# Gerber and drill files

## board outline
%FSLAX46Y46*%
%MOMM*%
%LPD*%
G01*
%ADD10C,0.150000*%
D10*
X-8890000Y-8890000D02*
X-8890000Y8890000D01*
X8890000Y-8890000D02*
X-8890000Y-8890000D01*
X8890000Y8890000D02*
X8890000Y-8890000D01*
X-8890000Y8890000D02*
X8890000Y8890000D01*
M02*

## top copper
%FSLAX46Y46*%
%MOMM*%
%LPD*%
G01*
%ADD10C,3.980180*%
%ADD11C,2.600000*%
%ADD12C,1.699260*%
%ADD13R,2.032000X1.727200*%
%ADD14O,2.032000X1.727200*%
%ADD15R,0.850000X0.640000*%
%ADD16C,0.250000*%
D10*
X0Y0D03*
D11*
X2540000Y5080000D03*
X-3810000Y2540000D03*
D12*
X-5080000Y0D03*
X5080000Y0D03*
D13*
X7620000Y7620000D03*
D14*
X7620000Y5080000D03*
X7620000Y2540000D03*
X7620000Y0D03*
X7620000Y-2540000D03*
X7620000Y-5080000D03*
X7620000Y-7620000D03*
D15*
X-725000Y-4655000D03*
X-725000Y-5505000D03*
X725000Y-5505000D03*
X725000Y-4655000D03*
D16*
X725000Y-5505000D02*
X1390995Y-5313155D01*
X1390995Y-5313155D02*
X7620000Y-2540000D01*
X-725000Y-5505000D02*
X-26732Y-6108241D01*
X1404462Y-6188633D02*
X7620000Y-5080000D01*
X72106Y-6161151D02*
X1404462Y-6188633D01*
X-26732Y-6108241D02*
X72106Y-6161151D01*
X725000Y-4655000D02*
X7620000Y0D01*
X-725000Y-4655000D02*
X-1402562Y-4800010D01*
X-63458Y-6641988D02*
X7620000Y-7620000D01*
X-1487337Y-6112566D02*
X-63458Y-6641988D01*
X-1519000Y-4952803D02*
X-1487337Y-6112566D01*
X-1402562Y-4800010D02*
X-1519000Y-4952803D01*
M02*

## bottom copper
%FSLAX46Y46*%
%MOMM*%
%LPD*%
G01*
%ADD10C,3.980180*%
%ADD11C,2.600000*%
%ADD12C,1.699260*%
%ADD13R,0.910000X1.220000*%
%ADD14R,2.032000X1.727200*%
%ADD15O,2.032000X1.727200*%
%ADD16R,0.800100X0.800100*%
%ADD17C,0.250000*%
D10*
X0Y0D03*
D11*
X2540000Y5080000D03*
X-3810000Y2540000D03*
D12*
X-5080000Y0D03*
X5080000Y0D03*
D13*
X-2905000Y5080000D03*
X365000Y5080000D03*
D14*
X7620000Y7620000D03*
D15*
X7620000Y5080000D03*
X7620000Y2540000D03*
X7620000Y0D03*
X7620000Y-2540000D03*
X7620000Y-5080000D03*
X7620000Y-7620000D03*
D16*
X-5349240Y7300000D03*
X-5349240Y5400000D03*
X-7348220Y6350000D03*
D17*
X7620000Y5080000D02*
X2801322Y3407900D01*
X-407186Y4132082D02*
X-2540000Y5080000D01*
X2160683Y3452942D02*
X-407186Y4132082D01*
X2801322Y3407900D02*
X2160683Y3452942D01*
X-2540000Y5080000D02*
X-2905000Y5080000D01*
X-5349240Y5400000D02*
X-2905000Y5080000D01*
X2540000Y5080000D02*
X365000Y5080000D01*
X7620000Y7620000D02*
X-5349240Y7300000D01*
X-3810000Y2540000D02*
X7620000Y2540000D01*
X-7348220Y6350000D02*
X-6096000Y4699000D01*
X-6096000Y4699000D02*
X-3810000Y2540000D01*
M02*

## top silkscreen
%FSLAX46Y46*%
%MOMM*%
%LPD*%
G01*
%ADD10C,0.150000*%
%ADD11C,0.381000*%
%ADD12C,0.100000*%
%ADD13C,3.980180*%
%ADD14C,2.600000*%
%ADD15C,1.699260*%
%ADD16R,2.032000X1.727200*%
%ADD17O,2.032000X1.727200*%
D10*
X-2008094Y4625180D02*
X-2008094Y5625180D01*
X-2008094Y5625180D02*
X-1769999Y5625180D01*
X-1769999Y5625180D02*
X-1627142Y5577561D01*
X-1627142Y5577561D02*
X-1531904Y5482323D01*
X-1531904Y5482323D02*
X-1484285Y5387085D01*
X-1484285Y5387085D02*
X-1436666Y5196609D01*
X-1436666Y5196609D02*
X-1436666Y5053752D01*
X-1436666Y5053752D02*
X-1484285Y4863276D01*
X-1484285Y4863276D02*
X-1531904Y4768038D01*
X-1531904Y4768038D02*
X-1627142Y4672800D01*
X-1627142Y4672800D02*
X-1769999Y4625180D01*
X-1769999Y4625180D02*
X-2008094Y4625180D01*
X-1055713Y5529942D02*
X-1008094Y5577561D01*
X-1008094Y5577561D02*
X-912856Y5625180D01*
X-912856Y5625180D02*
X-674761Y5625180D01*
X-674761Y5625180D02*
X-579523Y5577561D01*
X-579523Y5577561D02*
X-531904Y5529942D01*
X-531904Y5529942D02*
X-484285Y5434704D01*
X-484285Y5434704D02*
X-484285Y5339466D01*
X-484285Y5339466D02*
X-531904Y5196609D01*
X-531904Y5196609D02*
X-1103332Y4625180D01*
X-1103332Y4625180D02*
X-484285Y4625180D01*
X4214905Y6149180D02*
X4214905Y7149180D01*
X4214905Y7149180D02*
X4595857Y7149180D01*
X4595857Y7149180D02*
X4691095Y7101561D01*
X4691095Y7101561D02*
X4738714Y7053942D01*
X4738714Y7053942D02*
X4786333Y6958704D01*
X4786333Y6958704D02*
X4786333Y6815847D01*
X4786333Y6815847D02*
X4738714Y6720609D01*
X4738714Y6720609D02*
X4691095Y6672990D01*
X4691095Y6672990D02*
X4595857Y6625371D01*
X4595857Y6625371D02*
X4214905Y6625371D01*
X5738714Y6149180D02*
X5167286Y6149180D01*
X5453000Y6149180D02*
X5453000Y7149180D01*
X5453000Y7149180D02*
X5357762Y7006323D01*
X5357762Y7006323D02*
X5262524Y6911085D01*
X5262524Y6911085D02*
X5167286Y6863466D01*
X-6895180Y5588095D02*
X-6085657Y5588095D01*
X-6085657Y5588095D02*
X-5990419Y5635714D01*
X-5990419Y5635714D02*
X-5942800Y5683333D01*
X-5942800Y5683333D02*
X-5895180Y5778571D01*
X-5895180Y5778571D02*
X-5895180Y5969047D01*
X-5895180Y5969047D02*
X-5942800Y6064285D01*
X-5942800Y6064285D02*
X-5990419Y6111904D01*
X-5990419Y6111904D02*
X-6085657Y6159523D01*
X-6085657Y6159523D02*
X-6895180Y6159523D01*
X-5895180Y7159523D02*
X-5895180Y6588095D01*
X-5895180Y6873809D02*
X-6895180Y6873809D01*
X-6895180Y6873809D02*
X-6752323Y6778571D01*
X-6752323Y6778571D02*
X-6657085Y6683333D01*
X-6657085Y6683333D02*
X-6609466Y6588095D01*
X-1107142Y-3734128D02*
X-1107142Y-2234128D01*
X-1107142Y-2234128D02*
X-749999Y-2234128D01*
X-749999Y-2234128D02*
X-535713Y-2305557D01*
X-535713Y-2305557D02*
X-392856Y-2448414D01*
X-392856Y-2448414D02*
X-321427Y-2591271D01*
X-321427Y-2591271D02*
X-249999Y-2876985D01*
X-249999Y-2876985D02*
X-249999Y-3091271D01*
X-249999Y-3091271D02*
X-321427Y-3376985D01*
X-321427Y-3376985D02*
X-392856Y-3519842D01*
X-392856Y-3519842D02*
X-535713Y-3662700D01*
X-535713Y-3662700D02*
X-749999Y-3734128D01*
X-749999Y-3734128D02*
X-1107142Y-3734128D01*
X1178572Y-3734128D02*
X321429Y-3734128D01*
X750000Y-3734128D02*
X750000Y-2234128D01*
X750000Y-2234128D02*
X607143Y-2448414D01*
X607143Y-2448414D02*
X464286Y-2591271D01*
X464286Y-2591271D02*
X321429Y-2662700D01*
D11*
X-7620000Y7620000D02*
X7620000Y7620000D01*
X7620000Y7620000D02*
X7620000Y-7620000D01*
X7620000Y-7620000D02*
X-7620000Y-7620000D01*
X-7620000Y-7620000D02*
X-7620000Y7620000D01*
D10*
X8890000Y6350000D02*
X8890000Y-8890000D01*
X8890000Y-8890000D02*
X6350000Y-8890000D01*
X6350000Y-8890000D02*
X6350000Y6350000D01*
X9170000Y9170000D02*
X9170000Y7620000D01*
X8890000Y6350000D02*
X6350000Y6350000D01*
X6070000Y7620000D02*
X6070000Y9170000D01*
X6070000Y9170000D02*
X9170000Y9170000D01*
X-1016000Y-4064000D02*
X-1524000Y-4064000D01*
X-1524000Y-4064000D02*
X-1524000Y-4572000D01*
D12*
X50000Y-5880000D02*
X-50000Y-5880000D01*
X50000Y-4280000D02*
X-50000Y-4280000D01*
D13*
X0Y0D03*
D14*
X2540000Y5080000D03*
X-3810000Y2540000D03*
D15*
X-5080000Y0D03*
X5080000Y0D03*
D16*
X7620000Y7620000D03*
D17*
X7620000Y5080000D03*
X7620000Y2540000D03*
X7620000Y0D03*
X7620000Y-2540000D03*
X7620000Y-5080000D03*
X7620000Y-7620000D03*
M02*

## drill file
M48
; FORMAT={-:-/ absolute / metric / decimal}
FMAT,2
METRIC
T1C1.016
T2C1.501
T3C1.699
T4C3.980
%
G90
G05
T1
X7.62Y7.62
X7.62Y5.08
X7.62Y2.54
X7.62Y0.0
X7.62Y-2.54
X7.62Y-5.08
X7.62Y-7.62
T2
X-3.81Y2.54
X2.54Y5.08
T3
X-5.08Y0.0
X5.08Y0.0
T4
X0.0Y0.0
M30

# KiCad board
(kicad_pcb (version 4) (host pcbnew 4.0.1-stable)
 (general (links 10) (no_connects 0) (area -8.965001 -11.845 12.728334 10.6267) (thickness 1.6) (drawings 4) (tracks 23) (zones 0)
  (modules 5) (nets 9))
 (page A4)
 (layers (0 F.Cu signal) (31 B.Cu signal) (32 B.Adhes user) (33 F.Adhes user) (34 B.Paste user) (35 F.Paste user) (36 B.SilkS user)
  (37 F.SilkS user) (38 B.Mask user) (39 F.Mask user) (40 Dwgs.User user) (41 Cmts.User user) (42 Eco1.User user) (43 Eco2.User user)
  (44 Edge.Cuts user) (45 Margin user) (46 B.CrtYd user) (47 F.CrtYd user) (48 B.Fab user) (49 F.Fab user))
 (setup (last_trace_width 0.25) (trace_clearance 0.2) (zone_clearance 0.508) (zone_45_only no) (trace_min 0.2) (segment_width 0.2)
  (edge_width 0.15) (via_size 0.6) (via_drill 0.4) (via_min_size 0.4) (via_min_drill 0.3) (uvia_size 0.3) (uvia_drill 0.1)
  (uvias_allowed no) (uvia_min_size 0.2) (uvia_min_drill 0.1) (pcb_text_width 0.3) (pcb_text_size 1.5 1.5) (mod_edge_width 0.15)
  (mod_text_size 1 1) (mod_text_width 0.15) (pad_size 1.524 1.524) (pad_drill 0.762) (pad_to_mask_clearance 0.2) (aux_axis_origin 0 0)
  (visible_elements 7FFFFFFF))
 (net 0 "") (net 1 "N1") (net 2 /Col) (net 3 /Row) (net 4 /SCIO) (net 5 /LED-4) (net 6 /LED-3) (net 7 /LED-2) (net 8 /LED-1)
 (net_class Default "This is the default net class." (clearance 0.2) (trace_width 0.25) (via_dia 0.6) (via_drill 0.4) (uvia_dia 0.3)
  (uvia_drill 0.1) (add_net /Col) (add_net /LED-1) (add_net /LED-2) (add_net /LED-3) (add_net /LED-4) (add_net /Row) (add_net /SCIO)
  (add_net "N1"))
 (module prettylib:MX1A (layer F.Cu) (at 0 0)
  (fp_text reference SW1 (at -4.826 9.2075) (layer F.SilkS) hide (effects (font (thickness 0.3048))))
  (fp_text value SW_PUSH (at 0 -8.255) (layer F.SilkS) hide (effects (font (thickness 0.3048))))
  (fp_line (start -7.62 -7.62) (end 7.62 -7.62) (layer F.SilkS) (width 0.381))
  (fp_line (start 7.62 -7.62) (end 7.62 7.62) (layer F.SilkS) (width 0.381))
  (fp_line (start 7.62 7.62) (end -7.62 7.62) (layer F.SilkS) (width 0.381))
  (fp_line (start -7.62 7.62) (end -7.62 -7.62) (layer F.SilkS) (width 0.381))
  (pad 0 thru_hole circle (at 0 0) (size 3.98018 3.98018) (drill 3.98018) (layers *.Cu *.Mask F.SilkS))
  (pad 2 thru_hole circle (at 2.54 -5.08) (size 2.6 2.6) (drill 1.5011) (layers *.Cu *.Mask F.SilkS) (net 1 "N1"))
  (pad 1 thru_hole circle (at -3.81 -2.54) (size 2.6 2.6) (drill 1.5011) (layers *.Cu *.Mask F.SilkS) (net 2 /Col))
  (pad "" thru_hole circle (at -5.08 0) (size 1.69926 1.69926) (drill 1.69926) (layers *.Cu *.Mask F.SilkS))
  (pad "" thru_hole circle (at 5.08 0) (size 1.69926 1.69926) (drill 1.69926) (layers *.Cu *.Mask F.SilkS)))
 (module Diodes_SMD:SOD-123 (layer B.Cu) (at -1.27 -5.08)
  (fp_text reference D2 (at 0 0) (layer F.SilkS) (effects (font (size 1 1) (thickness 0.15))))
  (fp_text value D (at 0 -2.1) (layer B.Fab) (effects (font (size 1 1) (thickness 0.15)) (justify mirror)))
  (pad 1 smd rect (at -1.635 0) (size 0.91 1.22) (layers B.Cu B.Paste B.Mask) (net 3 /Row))
  (pad 2 smd rect (at 1.635 0) (size 0.91 1.22) (layers B.Cu B.Paste B.Mask) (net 1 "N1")))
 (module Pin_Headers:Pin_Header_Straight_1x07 (layer F.Cu) (at 7.62 -7.62)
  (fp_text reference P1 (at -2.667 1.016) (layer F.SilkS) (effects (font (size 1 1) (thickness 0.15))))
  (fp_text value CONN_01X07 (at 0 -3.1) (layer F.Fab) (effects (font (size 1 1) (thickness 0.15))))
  (fp_line (start 1.27 1.27) (end 1.27 16.51) (layer F.SilkS) (width 0.15))
  (fp_line (start 1.27 16.51) (end -1.27 16.51) (layer F.SilkS) (width 0.15))
  (fp_line (start -1.27 16.51) (end -1.27 1.27) (layer F.SilkS) (width 0.15))
  (fp_line (start 1.55 -1.55) (end 1.55 0) (layer F.SilkS) (width 0.15))
  (fp_line (start 1.27 1.27) (end -1.27 1.27) (layer F.SilkS) (width 0.15))
  (fp_line (start -1.55 0) (end -1.55 -1.55) (layer F.SilkS) (width 0.15))
  (fp_line (start -1.55 -1.55) (end 1.55 -1.55) (layer F.SilkS) (width 0.15))
  (pad 1 thru_hole rect (at 0 0) (size 2.032 1.7272) (drill 1.016) (layers *.Cu *.Mask F.SilkS) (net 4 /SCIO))
  (pad 2 thru_hole oval (at 0 2.54) (size 2.032 1.7272) (drill 1.016) (layers *.Cu *.Mask F.SilkS) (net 3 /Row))
  (pad 3 thru_hole oval (at 0 5.08) (size 2.032 1.7272) (drill 1.016) (layers *.Cu *.Mask F.SilkS) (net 2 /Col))
  (pad 4 thru_hole oval (at 0 7.62) (size 2.032 1.7272) (drill 1.016) (layers *.Cu *.Mask F.SilkS) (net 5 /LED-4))
  (pad 5 thru_hole oval (at 0 10.16) (size 2.032 1.7272) (drill 1.016) (layers *.Cu *.Mask F.SilkS) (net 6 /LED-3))
  (pad 6 thru_hole oval (at 0 12.7) (size 2.032 1.7272) (drill 1.016) (layers *.Cu *.Mask F.SilkS) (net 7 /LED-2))
  (pad 7 thru_hole oval (at 0 15.24) (size 2.032 1.7272) (drill 1.016) (layers *.Cu *.Mask F.SilkS) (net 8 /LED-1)))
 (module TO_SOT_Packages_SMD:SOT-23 (layer B.Cu) (at -6.35 -6.35 270)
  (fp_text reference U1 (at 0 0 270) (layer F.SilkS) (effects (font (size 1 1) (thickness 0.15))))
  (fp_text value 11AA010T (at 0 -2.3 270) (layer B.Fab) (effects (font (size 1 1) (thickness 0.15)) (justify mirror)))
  (pad 1 smd rect (at -0.95 -1.00076 270) (size 0.8001 0.8001) (layers B.Cu B.Paste B.Mask) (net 4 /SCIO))
  (pad 2 smd rect (at 0.95 -1.00076 270) (size 0.8001 0.8001) (layers B.Cu B.Paste B.Mask) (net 3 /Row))
  (pad 3 smd rect (at 0 0.99822 270) (size 0.8001 0.8001) (layers B.Cu B.Paste B.Mask) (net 2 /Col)))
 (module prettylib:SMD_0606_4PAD (layer F.Cu) (at 0 5.08 270)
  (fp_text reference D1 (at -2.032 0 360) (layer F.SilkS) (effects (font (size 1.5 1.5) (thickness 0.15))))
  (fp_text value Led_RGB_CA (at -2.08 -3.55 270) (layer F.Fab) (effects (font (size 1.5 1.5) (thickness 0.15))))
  (fp_line (start -1.016 1.016) (end -1.016 1.524) (layer F.SilkS) (width 0.15))
  (fp_line (start -1.016 1.524) (end -0.508 1.524) (layer F.SilkS) (width 0.15))
  (fp_line (start 0.8 -0.05) (end 0.8 0.05) (layer F.SilkS) (width 0.1))
  (fp_line (start -0.8 -0.05) (end -0.8 0.05) (layer F.SilkS) (width 0.1))
  (pad 1 smd rect (at -0.425 0.725 270) (size 0.64 0.85) (layers F.Cu F.Paste F.Mask) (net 8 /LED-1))
  (pad 2 smd rect (at 0.425 0.725 270) (size 0.64 0.85) (layers F.Cu F.Paste F.Mask) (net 7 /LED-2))
  (pad 3 smd rect (at 0.425 -0.725 270) (size 0.64 0.85) (layers F.Cu F.Paste F.Mask) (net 6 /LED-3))
  (pad 4 smd rect (at -0.425 -0.725 270) (size 0.64 0.85) (layers F.Cu F.Paste F.Mask) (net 5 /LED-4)))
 (gr_line (start -8.89 8.89) (end -8.89 -8.89) (angle 90) (layer Edge.Cuts) (width 0.15))
 (gr_line (start 8.89 8.89) (end -8.89 8.89) (angle 90) (layer Edge.Cuts) (width 0.15))
 (gr_line (start 8.89 -8.89) (end 8.89 8.89) (angle 90) (layer Edge.Cuts) (width 0.15))
 (gr_line (start -8.89 -8.89) (end 8.89 -8.89) (angle 90) (layer Edge.Cuts) (width 0.15))
 (segment (start 7.62 -5.08) (end 2.801322 -3.4079) (width 0.25) (layer B.Cu) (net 3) (status 10))
 (segment (start -0.407186 -4.132082) (end -2.54 -5.08) (width 0.25) (layer B.Cu) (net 3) (status 20))
 (segment (start 2.160683 -3.452942) (end -0.407186 -4.132082) (width 0.25) (layer B.Cu) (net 3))
 (segment (start 2.801322 -3.4079) (end 2.160683 -3.452942) (width 0.25) (layer B.Cu) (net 3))
 (segment (start -2.54 -5.08) (end -2.905 -5.08) (width 0.25) (layer B.Cu) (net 3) (status 30))
 (segment (start -5.34924 -5.4) (end -2.905 -5.08) (width 0.25) (layer B.Cu) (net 3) (status 30))
 (segment (start 2.54 -5.08) (end 0.365 -5.08) (width 0.25) (layer B.Cu) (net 1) (status 30))
 (segment (start 7.62 -7.62) (end -5.34924 -7.3) (width 0.25) (layer B.Cu) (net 4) (status 30))
 (segment (start -3.81 -2.54) (end 7.62 -2.54) (width 0.25) (layer B.Cu) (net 2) (status 30))
 (segment (start -7.34822 -6.35) (end -6.096 -4.699) (width 0.25) (layer B.Cu) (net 2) (status 10))
 (segment (start -6.096 -4.699) (end -3.81 -2.54) (width 0.25) (layer B.Cu) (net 2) (status 20))
 (segment (start 0.725 5.505) (end 1.390995 5.313155) (width 0.25) (layer F.Cu) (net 6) (status 10))
 (segment (start 1.390995 5.313155) (end 7.62 2.54) (width 0.25) (layer F.Cu) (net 6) (status 20))
 (segment (start -0.725 5.505) (end -0.026732 6.108241) (width 0.25) (layer F.Cu) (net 7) (status 400010))
 (segment (start 1.404462 6.188633) (end 7.62 5.08) (width 0.25) (layer F.Cu) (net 7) (status 800020))
 (segment (start 0.072106 6.161151) (end 1.404462 6.188633) (width 0.25) (layer F.Cu) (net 7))
 (segment (start -0.026732 6.108241) (end 0.072106 6.161151) (width 0.25) (layer F.Cu) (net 7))
 (segment (start 0.725 4.655) (end 7.62 0) (width 0.25) (layer F.Cu) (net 5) (status 30))
 (segment (start -0.725 4.655) (end -1.402562 4.80001) (width 0.25) (layer F.Cu) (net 8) (status 10))
 (segment (start -0.063458 6.641988) (end 7.62 7.62) (width 0.25) (layer F.Cu) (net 8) (status 800020))
 (segment (start -1.487337 6.112566) (end -0.063458 6.641988) (width 0.25) (layer F.Cu) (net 8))
 (segment (start -1.519 4.952803) (end -1.487337 6.112566) (width 0.25) (layer F.Cu) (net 8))
 (segment (start -1.402562 4.80001) (end -1.519 4.952803) (width 0.25) (layer F.Cu) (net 8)))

